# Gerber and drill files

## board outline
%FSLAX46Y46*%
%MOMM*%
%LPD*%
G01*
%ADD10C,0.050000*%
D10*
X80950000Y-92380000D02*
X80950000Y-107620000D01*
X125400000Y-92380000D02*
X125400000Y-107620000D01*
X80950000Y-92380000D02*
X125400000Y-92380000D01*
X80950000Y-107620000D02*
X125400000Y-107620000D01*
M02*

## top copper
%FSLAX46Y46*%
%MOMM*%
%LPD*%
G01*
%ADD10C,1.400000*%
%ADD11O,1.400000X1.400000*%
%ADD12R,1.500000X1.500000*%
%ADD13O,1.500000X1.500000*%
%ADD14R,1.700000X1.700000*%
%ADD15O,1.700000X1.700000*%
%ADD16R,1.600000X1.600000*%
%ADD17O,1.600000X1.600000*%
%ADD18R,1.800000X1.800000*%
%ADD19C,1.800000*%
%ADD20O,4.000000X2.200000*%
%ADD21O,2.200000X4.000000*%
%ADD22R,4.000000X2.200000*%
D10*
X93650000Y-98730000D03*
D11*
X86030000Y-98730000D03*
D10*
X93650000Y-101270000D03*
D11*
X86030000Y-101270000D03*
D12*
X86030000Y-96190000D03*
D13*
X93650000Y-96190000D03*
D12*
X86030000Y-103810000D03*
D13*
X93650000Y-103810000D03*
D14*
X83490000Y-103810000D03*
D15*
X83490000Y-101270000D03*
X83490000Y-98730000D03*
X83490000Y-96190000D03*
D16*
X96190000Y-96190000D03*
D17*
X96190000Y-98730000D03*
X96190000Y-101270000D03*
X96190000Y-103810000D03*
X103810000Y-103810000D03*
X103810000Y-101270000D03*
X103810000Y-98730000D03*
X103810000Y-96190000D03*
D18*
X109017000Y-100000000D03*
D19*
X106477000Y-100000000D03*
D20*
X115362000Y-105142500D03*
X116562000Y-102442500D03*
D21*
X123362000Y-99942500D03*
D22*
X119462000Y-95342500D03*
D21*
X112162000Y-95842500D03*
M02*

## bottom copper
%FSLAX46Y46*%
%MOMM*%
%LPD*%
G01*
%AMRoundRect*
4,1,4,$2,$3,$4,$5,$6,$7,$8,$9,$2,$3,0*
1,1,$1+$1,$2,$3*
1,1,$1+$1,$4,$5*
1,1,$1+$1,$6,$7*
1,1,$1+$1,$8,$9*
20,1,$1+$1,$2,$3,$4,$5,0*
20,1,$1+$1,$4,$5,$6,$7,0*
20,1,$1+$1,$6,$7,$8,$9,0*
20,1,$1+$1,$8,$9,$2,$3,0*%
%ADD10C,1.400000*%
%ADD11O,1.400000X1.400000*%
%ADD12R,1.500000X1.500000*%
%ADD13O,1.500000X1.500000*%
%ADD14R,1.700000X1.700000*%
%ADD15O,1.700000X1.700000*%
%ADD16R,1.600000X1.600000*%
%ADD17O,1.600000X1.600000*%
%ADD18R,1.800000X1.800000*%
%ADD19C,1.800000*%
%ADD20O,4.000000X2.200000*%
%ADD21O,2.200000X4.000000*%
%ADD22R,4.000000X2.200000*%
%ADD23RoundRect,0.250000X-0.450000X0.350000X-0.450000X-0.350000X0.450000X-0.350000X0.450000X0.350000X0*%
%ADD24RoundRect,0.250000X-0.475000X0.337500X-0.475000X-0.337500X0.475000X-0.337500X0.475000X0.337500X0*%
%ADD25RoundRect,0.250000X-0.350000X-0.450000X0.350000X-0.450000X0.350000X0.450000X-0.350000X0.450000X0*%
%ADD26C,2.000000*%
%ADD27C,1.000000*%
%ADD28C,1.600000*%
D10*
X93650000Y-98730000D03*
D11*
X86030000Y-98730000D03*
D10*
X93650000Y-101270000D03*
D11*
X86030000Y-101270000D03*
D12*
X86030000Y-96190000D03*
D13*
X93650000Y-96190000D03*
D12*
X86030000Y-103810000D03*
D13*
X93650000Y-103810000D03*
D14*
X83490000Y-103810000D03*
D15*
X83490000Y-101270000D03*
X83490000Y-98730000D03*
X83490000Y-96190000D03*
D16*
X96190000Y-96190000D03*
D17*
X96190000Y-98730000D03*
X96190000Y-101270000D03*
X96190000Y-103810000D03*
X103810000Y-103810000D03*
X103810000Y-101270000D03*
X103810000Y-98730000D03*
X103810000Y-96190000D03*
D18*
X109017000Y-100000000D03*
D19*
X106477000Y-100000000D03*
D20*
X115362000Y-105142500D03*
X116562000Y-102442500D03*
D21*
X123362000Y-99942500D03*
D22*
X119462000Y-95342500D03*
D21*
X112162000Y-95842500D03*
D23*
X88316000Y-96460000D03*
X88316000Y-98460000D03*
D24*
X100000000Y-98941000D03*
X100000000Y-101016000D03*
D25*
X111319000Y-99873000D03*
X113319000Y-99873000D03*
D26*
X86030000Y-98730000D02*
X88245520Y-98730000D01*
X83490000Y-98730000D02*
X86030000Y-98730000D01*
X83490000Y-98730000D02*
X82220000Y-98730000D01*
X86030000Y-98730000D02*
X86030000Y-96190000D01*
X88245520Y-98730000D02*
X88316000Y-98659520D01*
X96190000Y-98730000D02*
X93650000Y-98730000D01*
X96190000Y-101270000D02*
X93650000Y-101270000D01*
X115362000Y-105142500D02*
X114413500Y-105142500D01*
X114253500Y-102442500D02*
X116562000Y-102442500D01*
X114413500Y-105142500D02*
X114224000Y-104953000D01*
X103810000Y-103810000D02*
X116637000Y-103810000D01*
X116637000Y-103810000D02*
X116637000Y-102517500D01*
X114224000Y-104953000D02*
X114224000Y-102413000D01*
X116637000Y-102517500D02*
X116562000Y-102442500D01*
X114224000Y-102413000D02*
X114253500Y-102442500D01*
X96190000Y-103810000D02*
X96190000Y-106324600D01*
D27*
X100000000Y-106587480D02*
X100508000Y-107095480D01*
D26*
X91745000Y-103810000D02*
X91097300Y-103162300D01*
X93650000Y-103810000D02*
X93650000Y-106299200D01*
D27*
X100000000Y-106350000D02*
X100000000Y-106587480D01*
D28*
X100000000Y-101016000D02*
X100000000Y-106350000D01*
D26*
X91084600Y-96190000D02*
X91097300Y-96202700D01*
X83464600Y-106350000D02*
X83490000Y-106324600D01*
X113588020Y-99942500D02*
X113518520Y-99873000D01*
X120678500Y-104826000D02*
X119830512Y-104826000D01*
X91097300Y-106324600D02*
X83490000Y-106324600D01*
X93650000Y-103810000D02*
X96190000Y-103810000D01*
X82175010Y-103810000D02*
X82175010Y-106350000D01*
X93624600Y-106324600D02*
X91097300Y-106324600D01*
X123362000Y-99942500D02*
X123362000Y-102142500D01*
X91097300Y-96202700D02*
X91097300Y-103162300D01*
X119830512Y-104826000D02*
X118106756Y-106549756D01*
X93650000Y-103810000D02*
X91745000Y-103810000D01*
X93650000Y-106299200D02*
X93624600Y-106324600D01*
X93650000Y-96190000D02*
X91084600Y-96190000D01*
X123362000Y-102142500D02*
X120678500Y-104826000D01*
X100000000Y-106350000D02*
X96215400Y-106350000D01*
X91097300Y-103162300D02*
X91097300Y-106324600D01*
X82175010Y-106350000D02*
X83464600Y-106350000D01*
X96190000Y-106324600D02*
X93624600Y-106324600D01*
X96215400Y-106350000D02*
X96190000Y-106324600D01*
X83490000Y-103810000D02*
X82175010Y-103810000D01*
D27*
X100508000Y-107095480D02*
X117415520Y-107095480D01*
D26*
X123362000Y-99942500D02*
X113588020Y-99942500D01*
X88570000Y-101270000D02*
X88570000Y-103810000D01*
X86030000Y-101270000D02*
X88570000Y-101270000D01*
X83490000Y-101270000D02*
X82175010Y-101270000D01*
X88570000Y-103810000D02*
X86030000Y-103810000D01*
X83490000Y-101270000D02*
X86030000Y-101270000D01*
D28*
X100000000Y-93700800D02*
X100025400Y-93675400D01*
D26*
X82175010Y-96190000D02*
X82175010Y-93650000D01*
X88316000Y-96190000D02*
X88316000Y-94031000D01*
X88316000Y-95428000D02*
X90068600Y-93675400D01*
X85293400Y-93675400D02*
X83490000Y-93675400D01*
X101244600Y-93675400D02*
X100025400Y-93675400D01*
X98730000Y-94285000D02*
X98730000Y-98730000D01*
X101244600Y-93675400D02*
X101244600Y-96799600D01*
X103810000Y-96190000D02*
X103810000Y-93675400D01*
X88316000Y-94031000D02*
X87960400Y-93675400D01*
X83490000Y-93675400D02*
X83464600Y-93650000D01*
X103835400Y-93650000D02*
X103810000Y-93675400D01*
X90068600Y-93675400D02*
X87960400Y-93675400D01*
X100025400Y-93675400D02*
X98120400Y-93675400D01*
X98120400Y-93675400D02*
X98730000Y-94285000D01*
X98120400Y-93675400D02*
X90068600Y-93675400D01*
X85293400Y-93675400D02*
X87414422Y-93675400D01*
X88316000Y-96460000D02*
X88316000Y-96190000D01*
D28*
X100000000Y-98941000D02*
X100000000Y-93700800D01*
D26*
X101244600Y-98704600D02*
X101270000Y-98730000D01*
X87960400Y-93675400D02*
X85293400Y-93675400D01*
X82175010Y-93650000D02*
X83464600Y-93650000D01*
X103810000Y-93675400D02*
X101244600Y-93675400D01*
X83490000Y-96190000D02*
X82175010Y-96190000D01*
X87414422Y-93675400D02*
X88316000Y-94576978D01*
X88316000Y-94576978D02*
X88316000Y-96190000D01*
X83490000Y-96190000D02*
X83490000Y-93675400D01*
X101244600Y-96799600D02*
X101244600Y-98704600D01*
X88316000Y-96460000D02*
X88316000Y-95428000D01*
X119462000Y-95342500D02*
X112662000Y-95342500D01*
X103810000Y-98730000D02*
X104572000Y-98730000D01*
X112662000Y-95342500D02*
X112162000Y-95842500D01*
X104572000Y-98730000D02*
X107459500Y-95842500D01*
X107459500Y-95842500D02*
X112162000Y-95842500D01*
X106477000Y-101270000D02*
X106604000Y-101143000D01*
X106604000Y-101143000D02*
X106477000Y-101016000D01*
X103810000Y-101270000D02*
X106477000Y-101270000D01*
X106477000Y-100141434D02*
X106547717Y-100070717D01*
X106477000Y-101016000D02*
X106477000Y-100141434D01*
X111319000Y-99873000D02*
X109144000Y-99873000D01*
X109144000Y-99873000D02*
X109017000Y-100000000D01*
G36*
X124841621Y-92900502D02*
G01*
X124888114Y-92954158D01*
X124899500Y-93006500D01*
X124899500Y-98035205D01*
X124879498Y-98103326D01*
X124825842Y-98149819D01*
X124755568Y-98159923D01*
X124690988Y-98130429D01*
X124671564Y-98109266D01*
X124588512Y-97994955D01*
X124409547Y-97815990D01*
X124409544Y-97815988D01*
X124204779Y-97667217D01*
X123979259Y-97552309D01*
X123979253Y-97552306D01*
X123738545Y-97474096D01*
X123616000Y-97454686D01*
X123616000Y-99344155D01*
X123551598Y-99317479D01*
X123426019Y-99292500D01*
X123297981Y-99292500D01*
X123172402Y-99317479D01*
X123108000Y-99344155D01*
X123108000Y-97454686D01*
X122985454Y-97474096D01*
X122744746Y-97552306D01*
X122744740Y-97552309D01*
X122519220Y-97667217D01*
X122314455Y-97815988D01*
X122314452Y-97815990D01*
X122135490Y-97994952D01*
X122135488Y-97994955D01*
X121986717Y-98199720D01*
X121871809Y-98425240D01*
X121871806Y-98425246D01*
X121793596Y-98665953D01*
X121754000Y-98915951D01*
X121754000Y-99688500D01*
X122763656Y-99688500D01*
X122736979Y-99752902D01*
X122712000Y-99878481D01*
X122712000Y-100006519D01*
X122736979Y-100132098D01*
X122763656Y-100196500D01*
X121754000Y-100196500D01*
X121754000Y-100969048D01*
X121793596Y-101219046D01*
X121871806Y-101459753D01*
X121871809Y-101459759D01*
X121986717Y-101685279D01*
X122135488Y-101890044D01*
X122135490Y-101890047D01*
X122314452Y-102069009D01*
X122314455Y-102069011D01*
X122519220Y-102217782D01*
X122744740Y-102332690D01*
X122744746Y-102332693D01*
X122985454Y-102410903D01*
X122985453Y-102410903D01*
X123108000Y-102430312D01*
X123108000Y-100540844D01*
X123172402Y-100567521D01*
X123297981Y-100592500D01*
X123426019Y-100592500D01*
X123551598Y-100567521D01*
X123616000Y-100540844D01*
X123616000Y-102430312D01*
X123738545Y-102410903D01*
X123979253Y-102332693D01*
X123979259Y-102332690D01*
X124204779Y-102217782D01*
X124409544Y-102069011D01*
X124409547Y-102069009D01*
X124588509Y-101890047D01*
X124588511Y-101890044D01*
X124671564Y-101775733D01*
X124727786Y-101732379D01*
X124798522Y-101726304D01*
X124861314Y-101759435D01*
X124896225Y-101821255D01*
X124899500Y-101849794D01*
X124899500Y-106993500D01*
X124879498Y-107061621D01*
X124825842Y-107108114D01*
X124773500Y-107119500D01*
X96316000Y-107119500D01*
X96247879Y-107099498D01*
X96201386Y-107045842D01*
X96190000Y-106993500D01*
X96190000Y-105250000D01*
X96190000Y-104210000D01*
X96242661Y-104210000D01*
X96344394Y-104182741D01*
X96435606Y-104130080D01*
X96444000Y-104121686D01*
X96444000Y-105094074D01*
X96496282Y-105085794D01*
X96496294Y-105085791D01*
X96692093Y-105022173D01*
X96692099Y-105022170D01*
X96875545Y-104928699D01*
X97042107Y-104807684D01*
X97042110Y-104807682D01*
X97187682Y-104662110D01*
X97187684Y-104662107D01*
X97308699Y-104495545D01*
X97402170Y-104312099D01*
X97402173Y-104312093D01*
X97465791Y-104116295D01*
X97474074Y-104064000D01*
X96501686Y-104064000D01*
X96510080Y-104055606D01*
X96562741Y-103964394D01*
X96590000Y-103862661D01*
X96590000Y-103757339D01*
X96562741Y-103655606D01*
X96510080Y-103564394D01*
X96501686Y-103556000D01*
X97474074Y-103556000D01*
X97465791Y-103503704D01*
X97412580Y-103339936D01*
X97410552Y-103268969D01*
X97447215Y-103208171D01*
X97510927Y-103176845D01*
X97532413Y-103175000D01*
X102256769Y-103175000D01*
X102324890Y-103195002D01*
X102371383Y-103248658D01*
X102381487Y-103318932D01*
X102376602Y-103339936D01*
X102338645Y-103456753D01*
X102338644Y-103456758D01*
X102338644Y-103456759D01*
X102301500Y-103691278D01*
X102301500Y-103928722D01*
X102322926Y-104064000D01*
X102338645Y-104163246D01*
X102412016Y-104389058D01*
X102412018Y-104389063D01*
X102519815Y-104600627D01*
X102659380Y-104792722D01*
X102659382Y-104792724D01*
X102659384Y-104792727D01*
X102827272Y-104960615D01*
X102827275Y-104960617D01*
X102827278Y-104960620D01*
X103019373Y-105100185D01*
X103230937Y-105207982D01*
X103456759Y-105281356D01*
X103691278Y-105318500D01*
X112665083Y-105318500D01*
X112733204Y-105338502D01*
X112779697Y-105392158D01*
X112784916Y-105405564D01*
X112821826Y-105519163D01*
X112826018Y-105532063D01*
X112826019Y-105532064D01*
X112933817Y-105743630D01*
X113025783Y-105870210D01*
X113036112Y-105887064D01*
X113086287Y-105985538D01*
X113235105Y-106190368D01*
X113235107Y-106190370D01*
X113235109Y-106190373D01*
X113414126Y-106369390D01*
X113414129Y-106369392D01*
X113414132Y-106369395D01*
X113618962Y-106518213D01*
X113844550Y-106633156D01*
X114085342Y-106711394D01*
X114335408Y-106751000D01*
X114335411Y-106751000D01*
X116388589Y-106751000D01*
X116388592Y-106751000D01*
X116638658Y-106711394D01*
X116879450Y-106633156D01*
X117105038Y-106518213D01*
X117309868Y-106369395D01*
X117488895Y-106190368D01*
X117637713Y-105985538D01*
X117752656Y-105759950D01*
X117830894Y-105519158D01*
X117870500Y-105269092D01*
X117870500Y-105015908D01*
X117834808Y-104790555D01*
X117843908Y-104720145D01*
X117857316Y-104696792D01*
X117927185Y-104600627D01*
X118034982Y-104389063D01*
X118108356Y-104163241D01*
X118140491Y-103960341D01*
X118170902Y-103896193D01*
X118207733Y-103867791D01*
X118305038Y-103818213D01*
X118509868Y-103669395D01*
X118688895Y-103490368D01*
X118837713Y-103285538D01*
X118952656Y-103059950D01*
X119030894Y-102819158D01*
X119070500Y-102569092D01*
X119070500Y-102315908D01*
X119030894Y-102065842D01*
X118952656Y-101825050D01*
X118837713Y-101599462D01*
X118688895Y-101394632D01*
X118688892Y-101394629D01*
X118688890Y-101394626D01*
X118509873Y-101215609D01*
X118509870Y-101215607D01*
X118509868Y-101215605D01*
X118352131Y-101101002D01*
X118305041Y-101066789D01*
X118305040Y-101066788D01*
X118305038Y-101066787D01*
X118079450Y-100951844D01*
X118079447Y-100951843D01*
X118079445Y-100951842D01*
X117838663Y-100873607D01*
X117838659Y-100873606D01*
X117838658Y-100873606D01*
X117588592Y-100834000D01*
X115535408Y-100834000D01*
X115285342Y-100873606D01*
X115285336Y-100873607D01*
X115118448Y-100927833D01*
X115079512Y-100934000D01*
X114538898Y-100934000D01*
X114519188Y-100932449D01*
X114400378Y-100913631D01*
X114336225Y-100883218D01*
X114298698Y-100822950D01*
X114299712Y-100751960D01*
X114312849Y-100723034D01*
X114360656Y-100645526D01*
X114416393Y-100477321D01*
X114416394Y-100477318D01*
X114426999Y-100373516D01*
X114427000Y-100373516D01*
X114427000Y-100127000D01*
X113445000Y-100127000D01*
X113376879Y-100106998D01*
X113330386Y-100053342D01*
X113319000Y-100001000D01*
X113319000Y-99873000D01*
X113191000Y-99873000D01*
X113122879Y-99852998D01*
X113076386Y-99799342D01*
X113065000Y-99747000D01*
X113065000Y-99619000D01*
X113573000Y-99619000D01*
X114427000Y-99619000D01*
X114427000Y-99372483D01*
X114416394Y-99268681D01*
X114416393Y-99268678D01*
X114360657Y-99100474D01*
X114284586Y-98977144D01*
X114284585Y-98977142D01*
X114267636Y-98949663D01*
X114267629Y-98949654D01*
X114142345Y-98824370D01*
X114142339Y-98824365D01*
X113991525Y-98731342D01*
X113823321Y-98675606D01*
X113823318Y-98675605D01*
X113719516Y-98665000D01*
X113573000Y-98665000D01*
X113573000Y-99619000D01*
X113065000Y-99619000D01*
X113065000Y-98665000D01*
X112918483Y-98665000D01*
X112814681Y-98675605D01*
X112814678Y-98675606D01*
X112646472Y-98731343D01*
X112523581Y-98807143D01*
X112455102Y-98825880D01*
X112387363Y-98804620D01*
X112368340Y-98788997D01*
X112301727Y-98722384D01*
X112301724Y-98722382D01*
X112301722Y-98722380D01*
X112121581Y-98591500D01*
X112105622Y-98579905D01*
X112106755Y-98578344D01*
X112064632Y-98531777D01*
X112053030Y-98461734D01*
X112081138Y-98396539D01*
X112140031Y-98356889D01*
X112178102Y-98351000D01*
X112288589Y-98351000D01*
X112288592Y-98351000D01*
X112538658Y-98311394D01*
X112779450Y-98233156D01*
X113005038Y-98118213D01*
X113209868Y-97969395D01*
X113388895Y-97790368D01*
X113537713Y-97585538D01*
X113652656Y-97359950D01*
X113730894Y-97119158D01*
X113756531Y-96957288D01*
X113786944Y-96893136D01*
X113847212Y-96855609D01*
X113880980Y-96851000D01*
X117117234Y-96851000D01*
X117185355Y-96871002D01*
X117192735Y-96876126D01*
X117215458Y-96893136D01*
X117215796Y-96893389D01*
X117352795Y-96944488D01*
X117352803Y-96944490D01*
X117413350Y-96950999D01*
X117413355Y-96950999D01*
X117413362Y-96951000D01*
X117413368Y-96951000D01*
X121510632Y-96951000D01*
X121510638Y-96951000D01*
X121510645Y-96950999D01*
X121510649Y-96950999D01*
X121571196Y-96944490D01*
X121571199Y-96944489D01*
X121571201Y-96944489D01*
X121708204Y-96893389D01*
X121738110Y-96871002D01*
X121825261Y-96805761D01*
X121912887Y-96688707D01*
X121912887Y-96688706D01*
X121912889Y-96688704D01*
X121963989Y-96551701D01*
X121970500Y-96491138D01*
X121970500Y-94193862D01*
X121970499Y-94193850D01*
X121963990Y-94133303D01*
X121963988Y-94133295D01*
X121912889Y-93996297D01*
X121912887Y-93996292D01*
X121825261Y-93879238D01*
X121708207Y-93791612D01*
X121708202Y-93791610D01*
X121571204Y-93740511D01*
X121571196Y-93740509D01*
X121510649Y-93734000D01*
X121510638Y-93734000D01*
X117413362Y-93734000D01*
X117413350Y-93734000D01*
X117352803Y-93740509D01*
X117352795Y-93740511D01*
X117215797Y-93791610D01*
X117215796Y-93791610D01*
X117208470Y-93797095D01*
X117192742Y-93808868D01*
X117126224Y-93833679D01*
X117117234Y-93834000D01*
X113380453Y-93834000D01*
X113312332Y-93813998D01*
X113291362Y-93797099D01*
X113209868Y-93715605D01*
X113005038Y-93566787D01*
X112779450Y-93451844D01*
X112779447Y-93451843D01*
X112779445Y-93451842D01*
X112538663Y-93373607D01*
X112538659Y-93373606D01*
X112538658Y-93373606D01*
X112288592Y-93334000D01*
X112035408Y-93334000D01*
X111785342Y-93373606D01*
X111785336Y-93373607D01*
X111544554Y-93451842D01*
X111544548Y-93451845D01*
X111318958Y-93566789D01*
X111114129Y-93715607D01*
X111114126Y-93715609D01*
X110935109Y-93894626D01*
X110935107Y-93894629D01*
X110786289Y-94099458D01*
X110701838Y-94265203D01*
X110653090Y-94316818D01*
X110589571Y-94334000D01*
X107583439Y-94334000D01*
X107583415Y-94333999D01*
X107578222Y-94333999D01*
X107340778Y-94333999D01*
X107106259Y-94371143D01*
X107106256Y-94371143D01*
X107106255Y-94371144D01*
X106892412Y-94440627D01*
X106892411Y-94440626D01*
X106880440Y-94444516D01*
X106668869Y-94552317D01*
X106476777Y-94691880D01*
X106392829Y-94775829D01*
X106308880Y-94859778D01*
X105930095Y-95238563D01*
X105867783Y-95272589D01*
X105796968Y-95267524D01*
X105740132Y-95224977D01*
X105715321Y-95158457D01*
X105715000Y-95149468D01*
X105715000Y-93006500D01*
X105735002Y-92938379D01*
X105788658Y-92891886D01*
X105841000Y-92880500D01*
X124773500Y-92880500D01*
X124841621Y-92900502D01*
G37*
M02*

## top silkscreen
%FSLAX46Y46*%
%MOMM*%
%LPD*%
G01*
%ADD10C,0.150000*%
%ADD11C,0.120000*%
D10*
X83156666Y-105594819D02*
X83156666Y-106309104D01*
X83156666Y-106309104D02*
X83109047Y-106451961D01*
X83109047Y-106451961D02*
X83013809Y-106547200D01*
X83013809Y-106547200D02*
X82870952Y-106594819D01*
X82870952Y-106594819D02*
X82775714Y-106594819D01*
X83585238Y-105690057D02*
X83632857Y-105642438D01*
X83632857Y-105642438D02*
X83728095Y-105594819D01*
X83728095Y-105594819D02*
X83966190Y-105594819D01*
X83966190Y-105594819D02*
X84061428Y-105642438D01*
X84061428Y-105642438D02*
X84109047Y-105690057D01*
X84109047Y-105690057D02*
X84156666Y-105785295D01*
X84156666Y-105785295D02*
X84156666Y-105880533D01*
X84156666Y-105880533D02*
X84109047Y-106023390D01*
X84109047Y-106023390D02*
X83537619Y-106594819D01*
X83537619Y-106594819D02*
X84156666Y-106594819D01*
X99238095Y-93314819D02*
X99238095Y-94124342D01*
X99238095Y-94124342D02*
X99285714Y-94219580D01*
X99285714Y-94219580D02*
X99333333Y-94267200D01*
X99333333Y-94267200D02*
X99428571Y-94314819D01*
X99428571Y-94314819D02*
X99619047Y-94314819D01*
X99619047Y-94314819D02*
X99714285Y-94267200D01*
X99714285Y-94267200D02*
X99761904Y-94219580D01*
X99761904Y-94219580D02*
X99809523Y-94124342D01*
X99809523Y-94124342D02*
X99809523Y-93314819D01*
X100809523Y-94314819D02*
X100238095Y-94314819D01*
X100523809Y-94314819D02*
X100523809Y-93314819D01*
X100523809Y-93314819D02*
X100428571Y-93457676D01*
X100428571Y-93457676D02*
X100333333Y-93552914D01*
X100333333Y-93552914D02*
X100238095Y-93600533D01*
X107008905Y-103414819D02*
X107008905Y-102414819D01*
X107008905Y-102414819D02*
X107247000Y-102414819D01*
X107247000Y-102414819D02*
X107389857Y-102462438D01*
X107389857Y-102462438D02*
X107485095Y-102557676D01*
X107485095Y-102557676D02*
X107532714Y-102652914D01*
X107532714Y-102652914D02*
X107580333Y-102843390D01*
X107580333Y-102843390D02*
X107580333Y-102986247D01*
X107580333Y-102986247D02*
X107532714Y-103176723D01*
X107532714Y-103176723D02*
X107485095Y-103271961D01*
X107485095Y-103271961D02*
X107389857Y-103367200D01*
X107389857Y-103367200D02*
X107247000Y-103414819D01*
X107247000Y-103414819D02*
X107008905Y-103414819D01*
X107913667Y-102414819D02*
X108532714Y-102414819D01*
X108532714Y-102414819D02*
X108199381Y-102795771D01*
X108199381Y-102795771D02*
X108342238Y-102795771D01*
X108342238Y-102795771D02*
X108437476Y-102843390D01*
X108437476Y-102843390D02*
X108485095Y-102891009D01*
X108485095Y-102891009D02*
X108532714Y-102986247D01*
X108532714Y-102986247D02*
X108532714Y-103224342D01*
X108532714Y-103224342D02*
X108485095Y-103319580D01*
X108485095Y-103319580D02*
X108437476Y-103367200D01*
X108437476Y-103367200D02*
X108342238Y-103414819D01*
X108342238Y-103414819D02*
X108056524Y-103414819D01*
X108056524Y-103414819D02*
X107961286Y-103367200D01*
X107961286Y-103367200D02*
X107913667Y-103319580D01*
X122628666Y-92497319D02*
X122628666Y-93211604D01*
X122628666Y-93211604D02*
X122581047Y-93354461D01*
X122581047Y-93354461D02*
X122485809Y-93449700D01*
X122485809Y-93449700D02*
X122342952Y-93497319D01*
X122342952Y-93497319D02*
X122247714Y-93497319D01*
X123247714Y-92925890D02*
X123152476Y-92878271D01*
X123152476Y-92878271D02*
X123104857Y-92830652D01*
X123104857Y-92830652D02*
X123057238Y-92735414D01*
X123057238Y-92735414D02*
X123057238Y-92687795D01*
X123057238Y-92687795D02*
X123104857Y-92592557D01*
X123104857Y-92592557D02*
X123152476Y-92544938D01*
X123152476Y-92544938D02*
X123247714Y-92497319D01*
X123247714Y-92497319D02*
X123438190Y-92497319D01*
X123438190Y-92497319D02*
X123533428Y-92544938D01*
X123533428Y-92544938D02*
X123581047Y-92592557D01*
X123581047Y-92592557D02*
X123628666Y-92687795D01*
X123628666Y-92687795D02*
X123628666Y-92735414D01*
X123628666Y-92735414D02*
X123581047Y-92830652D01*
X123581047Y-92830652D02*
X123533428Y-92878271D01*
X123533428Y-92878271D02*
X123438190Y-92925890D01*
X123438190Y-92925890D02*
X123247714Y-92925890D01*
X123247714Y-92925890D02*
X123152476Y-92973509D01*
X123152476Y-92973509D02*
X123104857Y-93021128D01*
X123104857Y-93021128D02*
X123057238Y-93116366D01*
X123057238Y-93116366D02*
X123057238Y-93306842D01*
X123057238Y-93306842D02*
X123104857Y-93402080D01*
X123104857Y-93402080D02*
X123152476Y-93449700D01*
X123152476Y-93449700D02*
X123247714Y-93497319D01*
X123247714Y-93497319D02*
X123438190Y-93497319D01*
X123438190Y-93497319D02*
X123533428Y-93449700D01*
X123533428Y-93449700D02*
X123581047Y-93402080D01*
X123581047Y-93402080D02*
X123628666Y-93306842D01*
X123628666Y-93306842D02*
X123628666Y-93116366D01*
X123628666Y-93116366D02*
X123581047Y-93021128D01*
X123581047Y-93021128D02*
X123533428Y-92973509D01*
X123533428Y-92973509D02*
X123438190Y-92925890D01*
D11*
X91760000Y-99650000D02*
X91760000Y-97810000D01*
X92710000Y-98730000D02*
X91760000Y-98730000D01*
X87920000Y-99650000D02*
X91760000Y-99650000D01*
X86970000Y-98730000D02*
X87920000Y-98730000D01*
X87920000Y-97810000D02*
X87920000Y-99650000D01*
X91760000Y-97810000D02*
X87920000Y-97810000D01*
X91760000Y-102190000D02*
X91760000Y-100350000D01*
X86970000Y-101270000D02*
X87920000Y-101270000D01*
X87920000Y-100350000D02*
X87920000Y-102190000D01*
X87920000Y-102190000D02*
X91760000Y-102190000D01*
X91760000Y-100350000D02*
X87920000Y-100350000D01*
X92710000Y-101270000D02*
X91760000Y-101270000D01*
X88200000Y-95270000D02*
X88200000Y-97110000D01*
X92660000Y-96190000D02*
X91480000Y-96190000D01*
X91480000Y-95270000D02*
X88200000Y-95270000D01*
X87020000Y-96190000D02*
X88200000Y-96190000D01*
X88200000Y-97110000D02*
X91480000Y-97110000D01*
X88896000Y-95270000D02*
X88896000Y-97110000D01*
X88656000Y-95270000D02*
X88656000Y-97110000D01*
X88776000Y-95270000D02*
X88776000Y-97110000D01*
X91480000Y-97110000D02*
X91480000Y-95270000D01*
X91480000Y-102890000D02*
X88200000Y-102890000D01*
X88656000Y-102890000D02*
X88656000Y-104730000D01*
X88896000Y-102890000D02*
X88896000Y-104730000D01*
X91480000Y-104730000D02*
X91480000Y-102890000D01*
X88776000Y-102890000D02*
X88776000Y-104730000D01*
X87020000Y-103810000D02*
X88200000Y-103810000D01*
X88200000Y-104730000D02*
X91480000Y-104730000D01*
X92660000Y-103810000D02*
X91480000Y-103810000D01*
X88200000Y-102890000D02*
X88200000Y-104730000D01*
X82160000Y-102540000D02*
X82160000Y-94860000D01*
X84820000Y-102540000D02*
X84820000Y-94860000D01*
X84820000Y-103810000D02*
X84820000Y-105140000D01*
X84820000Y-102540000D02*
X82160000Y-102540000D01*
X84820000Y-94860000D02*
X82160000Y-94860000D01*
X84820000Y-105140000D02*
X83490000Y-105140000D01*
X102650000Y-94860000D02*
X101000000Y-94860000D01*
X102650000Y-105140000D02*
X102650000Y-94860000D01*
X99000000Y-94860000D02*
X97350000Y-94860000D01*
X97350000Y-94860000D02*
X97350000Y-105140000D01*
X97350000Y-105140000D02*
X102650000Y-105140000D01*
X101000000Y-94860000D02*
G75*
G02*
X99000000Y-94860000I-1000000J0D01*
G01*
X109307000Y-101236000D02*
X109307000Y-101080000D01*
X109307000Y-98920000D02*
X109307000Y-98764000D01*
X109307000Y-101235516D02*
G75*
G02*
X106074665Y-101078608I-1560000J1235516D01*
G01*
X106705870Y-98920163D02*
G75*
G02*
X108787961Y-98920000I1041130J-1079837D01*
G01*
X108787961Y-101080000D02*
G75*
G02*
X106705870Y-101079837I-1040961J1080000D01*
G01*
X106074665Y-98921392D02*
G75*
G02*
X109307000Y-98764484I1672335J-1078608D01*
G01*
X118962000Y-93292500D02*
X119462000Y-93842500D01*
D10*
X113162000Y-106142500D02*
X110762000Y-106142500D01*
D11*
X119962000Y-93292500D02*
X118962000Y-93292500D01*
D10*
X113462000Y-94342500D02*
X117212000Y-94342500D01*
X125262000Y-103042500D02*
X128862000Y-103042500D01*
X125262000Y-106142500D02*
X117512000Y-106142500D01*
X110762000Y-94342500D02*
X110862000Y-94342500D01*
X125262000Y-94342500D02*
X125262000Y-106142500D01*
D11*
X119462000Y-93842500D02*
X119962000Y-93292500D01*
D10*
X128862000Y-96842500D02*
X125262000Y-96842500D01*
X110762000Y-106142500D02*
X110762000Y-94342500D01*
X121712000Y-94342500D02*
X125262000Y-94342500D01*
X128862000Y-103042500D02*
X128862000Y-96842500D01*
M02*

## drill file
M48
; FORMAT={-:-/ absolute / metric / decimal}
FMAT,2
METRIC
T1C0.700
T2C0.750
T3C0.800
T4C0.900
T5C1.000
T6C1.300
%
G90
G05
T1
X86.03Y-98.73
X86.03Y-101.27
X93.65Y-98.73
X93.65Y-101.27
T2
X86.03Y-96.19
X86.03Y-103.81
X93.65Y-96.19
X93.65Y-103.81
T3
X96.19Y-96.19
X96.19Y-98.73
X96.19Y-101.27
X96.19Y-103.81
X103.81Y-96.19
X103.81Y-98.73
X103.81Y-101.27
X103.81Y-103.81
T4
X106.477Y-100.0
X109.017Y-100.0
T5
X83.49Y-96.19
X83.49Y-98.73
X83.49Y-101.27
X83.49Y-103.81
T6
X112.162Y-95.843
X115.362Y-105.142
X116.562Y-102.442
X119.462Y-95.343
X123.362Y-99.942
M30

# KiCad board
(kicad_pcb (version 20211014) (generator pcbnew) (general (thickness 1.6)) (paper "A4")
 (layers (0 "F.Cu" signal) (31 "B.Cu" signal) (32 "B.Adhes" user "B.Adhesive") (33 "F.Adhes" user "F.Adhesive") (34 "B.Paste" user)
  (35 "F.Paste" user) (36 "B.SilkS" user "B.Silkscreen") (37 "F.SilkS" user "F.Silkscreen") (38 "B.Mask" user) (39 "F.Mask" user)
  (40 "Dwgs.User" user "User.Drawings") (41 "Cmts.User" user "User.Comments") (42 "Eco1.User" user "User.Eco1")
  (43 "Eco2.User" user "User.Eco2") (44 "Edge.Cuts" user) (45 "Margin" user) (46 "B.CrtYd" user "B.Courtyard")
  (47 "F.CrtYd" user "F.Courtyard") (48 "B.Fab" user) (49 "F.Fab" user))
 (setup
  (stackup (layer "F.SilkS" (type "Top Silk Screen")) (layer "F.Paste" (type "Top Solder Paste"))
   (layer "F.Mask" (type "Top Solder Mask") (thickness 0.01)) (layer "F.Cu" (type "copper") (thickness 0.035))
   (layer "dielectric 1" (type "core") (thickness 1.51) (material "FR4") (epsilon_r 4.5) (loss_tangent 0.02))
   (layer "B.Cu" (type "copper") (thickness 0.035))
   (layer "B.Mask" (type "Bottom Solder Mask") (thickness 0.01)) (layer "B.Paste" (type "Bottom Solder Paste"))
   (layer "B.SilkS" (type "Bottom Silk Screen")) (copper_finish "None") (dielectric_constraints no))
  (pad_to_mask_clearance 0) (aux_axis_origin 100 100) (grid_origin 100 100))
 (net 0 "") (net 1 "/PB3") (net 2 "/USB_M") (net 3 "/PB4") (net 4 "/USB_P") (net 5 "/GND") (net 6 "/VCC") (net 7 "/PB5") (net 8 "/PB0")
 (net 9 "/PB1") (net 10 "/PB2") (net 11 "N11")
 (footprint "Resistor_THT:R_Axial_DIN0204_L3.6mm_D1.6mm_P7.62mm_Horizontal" (layer "F.Cu") (at 93.65 98.73 180)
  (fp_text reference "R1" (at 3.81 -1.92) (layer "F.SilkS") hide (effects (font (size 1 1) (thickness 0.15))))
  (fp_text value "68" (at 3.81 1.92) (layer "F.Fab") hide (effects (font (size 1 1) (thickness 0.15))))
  (fp_line (start 1.89 -0.92) (end 1.89 0.92) (layer "F.SilkS") (width 0.12))
  (fp_line (start 0.94 0) (end 1.89 0) (layer "F.SilkS") (width 0.12))
  (fp_line (start 5.73 -0.92) (end 1.89 -0.92) (layer "F.SilkS") (width 0.12))
  (fp_line (start 6.68 0) (end 5.73 0) (layer "F.SilkS") (width 0.12))
  (fp_line (start 5.73 0.92) (end 5.73 -0.92) (layer "F.SilkS") (width 0.12))
  (fp_line (start 1.89 0.92) (end 5.73 0.92) (layer "F.SilkS") (width 0.12))
  (pad "1" thru_hole circle locked (at 0 0 180) (size 1.4 1.4) (drill 0.7) (layers *.Cu *.Mask) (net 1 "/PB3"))
  (pad "2" thru_hole oval locked (at 7.62 0 180) (size 1.4 1.4) (drill 0.7) (layers *.Cu *.Mask) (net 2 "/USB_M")))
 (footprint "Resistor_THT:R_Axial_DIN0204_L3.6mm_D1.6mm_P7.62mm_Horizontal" (layer "F.Cu") (at 93.65 101.27 180)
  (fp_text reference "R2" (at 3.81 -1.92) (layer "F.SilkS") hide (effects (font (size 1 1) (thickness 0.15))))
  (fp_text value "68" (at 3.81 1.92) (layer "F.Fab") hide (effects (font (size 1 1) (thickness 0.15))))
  (fp_line (start 1.89 -0.92) (end 1.89 0.92) (layer "F.SilkS") (width 0.12))
  (fp_line (start 6.68 0) (end 5.73 0) (layer "F.SilkS") (width 0.12))
  (fp_line (start 5.73 0.92) (end 5.73 -0.92) (layer "F.SilkS") (width 0.12))
  (fp_line (start 5.73 -0.92) (end 1.89 -0.92) (layer "F.SilkS") (width 0.12))
  (fp_line (start 1.89 0.92) (end 5.73 0.92) (layer "F.SilkS") (width 0.12))
  (fp_line (start 0.94 0) (end 1.89 0) (layer "F.SilkS") (width 0.12))
  (pad "1" thru_hole circle locked (at 0 0 180) (size 1.4 1.4) (drill 0.7) (layers *.Cu *.Mask) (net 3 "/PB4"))
  (pad "2" thru_hole oval locked (at 7.62 0 180) (size 1.4 1.4) (drill 0.7) (layers *.Cu *.Mask) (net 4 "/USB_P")))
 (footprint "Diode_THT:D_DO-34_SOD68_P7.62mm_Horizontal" (layer "F.Cu") (at 86.03 96.19)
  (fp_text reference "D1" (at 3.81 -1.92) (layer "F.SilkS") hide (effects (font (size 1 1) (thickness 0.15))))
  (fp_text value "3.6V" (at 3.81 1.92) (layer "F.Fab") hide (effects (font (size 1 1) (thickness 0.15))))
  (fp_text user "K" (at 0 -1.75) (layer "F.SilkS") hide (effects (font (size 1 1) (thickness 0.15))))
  (fp_line (start 2.17 -0.92) (end 2.17 0.92) (layer "F.SilkS") (width 0.12))
  (fp_line (start 6.63 0) (end 5.45 0) (layer "F.SilkS") (width 0.12))
  (fp_line (start 5.45 -0.92) (end 2.17 -0.92) (layer "F.SilkS") (width 0.12))
  (fp_line (start 0.99 0) (end 2.17 0) (layer "F.SilkS") (width 0.12))
  (fp_line (start 2.17 0.92) (end 5.45 0.92) (layer "F.SilkS") (width 0.12))
  (fp_line (start 2.866 -0.92) (end 2.866 0.92) (layer "F.SilkS") (width 0.12))
  (fp_line (start 2.626 -0.92) (end 2.626 0.92) (layer "F.SilkS") (width 0.12))
  (fp_line (start 2.746 -0.92) (end 2.746 0.92) (layer "F.SilkS") (width 0.12))
  (fp_line (start 5.45 0.92) (end 5.45 -0.92) (layer "F.SilkS") (width 0.12))
  (pad "1" thru_hole rect locked (at 0 0) (size 1.5 1.5) (drill 0.75) (layers *.Cu *.Mask) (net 2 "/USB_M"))
  (pad "2" thru_hole oval locked (at 7.62 0) (size 1.5 1.5) (drill 0.75) (layers *.Cu *.Mask) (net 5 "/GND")))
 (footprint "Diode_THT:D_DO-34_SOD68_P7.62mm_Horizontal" (layer "F.Cu") (at 86.03 103.81)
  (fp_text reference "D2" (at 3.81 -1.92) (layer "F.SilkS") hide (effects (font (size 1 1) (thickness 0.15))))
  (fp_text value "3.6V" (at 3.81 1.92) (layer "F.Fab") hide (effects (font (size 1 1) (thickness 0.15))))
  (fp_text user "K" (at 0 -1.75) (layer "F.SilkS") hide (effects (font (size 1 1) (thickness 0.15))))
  (fp_line (start 5.45 -0.92) (end 2.17 -0.92) (layer "F.SilkS") (width 0.12))
  (fp_line (start 2.626 -0.92) (end 2.626 0.92) (layer "F.SilkS") (width 0.12))
  (fp_line (start 2.866 -0.92) (end 2.866 0.92) (layer "F.SilkS") (width 0.12))
  (fp_line (start 5.45 0.92) (end 5.45 -0.92) (layer "F.SilkS") (width 0.12))
  (fp_line (start 2.746 -0.92) (end 2.746 0.92) (layer "F.SilkS") (width 0.12))
  (fp_line (start 0.99 0) (end 2.17 0) (layer "F.SilkS") (width 0.12))
  (fp_line (start 2.17 0.92) (end 5.45 0.92) (layer "F.SilkS") (width 0.12))
  (fp_line (start 6.63 0) (end 5.45 0) (layer "F.SilkS") (width 0.12))
  (fp_line (start 2.17 -0.92) (end 2.17 0.92) (layer "F.SilkS") (width 0.12))
  (pad "1" thru_hole rect locked (at 0 0) (size 1.5 1.5) (drill 0.75) (layers *.Cu *.Mask) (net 4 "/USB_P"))
  (pad "2" thru_hole oval locked (at 7.62 0) (size 1.5 1.5) (drill 0.75) (layers *.Cu *.Mask) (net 5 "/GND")))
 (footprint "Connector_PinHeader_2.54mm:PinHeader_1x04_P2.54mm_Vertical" (layer "F.Cu") (at 83.49 103.81 180)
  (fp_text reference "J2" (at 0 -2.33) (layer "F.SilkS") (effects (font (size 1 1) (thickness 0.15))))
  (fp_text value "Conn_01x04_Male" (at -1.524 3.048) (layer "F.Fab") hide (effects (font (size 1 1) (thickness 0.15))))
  (fp_line (start 1.33 1.27) (end 1.33 8.95) (layer "F.SilkS") (width 0.12))
  (fp_line (start -1.33 1.27) (end -1.33 8.95) (layer "F.SilkS") (width 0.12))
  (fp_line (start -1.33 0) (end -1.33 -1.33) (layer "F.SilkS") (width 0.12))
  (fp_line (start -1.33 1.27) (end 1.33 1.27) (layer "F.SilkS") (width 0.12))
  (fp_line (start -1.33 8.95) (end 1.33 8.95) (layer "F.SilkS") (width 0.12))
  (fp_line (start -1.33 -1.33) (end 0 -1.33) (layer "F.SilkS") (width 0.12))
  (pad "1" thru_hole rect locked (at 0 0 180) (size 1.7 1.7) (drill 1) (layers *.Cu *.Mask) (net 5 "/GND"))
  (pad "2" thru_hole oval locked (at 0 2.54 180) (size 1.7 1.7) (drill 1) (layers *.Cu *.Mask) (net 4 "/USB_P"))
  (pad "3" thru_hole oval locked (at 0 5.08 180) (size 1.7 1.7) (drill 1) (layers *.Cu *.Mask) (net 2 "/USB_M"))
  (pad "4" thru_hole oval locked (at 0 7.62 180) (size 1.7 1.7) (drill 1) (layers *.Cu *.Mask) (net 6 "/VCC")))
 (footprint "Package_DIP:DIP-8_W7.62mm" (layer "F.Cu") (at 96.19 96.19)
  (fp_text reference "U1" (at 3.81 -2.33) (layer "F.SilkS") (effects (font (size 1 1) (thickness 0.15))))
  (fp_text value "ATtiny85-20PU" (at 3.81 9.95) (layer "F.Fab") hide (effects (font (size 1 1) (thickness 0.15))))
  (fp_line (start 6.46 -1.33) (end 4.81 -1.33) (layer "F.SilkS") (width 0.12))
  (fp_line (start 6.46 8.95) (end 6.46 -1.33) (layer "F.SilkS") (width 0.12))
  (fp_line (start 2.81 -1.33) (end 1.16 -1.33) (layer "F.SilkS") (width 0.12))
  (fp_line (start 1.16 -1.33) (end 1.16 8.95) (layer "F.SilkS") (width 0.12))
  (fp_line (start 1.16 8.95) (end 6.46 8.95) (layer "F.SilkS") (width 0.12))
  (fp_arc (start 4.81 -1.33) (mid 3.81 -0.33) (end 2.81 -1.33) (layer "F.SilkS") (width 0.12))
  (pad "1" thru_hole rect locked (at 0 0) (size 1.6 1.6) (drill 0.8) (layers *.Cu *.Mask) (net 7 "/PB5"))
  (pad "2" thru_hole oval locked (at 0 2.54) (size 1.6 1.6) (drill 0.8) (layers *.Cu *.Mask) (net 1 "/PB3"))
  (pad "3" thru_hole oval locked (at 0 5.08) (size 1.6 1.6) (drill 0.8) (layers *.Cu *.Mask) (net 3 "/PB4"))
  (pad "4" thru_hole oval locked (at 0 7.62) (size 1.6 1.6) (drill 0.8) (layers *.Cu *.Mask) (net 5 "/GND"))
  (pad "5" thru_hole oval locked (at 7.62 7.62) (size 1.6 1.6) (drill 0.8) (layers *.Cu *.Mask) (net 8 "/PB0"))
  (pad "6" thru_hole oval locked (at 7.62 5.08) (size 1.6 1.6) (drill 0.8) (layers *.Cu *.Mask) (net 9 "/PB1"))
  (pad "7" thru_hole oval locked (at 7.62 2.54) (size 1.6 1.6) (drill 0.8) (layers *.Cu *.Mask) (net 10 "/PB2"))
  (pad "8" thru_hole oval locked (at 7.62 0) (size 1.6 1.6) (drill 0.8) (layers *.Cu *.Mask) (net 6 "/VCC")))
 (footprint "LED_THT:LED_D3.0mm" (layer "F.Cu") (at 109.017 100 180)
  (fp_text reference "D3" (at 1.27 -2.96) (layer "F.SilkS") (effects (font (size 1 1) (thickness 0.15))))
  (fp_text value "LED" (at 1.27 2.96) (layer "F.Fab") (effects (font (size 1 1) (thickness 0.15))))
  (fp_line (start -0.29 -1.236) (end -0.29 -1.08) (layer "F.SilkS") (width 0.12))
  (fp_line (start -0.29 1.08) (end -0.29 1.236) (layer "F.SilkS") (width 0.12))
  (fp_arc (start -0.29 -1.235516) (mid 1.366487 -1.987659) (end 2.942335 -1.078608) (layer "F.SilkS") (width 0.12))
  (fp_arc (start 2.31113 1.079837) (mid 1.270117 1.5) (end 0.229039 1.08) (layer "F.SilkS") (width 0.12))
  (fp_arc (start 0.229039 -1.08) (mid 1.270117 -1.5) (end 2.31113 -1.079837) (layer "F.SilkS") (width 0.12))
  (fp_arc (start 2.942335 1.078608) (mid 1.366487 1.987659) (end -0.29 1.235516) (layer "F.SilkS") (width 0.12))
  (pad "1" thru_hole rect (at 0 0 180) (size 1.8 1.8) (drill 0.9) (layers *.Cu *.Mask) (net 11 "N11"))
  (pad "2" thru_hole circle (at 2.54 0 180) (size 1.8 1.8) (drill 0.9) (layers *.Cu *.Mask) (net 9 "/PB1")))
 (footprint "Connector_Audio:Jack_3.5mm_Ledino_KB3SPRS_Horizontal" (layer "F.Cu") (at 119.462 95.3425 180)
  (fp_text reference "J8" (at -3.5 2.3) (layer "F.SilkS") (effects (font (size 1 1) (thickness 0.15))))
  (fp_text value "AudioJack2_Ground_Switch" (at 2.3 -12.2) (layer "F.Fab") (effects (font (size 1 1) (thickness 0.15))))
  (fp_line (start 0.5 2.05) (end 0 1.5) (layer "F.SilkS") (width 0.12))
  (fp_line (start 6.3 -10.8) (end 8.7 -10.8) (layer "F.SilkS") (width 0.15))
  (fp_line (start -0.5 2.05) (end 0.5 2.05) (layer "F.SilkS") (width 0.12))
  (fp_line (start 6 1) (end 2.25 1) (layer "F.SilkS") (width 0.15))
  (fp_line (start -5.8 -7.7) (end -9.4 -7.7) (layer "F.SilkS") (width 0.15))
  (fp_line (start -5.8 -10.8) (end 1.95 -10.8) (layer "F.SilkS") (width 0.15))
  (fp_line (start 8.7 1) (end 8.6 1) (layer "F.SilkS") (width 0.15))
  (fp_line (start -5.8 1) (end -5.8 -10.8) (layer "F.SilkS") (width 0.15))
  (fp_line (start 0 1.5) (end -0.5 2.05) (layer "F.SilkS") (width 0.12))
  (fp_line (start -9.4 -1.5) (end -5.8 -1.5) (layer "F.SilkS") (width 0.15))
  (fp_line (start 8.7 -10.8) (end 8.7 1) (layer "F.SilkS") (width 0.15))
  (fp_line (start -2.25 1) (end -5.8 1) (layer "F.SilkS") (width 0.15))
  (fp_line (start -9.4 -7.7) (end -9.4 -1.5) (layer "F.SilkS") (width 0.15))
  (pad "R" thru_hole oval (at 4.1 -9.8 180) (size 4 2.2) (drill 1.3) (layers *.Cu *.Mask) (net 8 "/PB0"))
  (pad "RN" thru_hole oval (at 2.9 -7.1 180) (size 4 2.2) (drill 1.3) (layers *.Cu *.Mask) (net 8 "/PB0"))
  (pad "S" thru_hole oval (at -3.9 -4.6 180) (size 2.2 4) (drill 1.3) (layers *.Cu *.Mask) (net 5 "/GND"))
  (pad "T" thru_hole rect (at 0 0 180) (size 4 2.2) (drill 1.3) (layers *.Cu *.Mask) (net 10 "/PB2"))
  (pad "TN" thru_hole oval (at 7.3 -0.5 270) (size 4 2.2) (drill 1.3) (layers *.Cu *.Mask) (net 10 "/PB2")))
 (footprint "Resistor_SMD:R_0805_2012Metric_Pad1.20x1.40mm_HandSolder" (layer "B.Cu") (at 88.316 97.46 -90)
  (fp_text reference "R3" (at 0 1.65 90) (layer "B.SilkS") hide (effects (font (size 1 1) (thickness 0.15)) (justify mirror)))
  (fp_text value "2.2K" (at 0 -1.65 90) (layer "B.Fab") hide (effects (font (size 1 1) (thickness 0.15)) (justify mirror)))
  (pad "1" smd roundrect locked (at -1 0 270) (size 1.2 1.4) (layers "B.Cu" "B.Paste" "B.Mask") (roundrect_rratio 0.2083333333)
   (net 6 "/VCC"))
  (pad "2" smd roundrect locked (at 1 0 270) (size 1.2 1.4) (layers "B.Cu" "B.Paste" "B.Mask") (roundrect_rratio 0.2083333333)
   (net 2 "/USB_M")))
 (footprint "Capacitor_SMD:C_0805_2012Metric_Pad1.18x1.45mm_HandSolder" (layer "B.Cu") (at 100 99.9785 -90)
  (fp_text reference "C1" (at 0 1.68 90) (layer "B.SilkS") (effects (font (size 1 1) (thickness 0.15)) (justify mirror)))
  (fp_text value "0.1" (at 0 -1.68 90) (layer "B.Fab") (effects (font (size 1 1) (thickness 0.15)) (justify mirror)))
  (pad "1" smd roundrect locked (at -1.0375 0 270) (size 1.175 1.45) (layers "B.Cu" "B.Paste" "B.Mask") (roundrect_rratio 0.2127659574)
   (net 6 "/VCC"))
  (pad "2" smd roundrect locked (at 1.0375 0 270) (size 1.175 1.45) (layers "B.Cu" "B.Paste" "B.Mask") (roundrect_rratio 0.2127659574)
   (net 5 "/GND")))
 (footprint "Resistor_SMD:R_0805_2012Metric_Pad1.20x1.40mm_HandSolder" (layer "B.Cu") (at 112.319 99.873)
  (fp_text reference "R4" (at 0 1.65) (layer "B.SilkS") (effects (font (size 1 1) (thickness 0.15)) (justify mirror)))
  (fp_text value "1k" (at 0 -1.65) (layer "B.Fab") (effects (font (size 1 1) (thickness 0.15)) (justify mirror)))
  (pad "1" smd roundrect (at -1 0) (size 1.2 1.4) (layers "B.Cu" "B.Paste" "B.Mask") (roundrect_rratio 0.208333) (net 11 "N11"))
  (pad "2" smd roundrect (at 1 0) (size 1.2 1.4) (layers "B.Cu" "B.Paste" "B.Mask") (roundrect_rratio 0.208333) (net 5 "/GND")))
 (gr_line (start 80.95 92.38) (end 80.95 107.62) (layer "Edge.Cuts") (width 0.05))
 (gr_line (start 125.4 92.38) (end 125.4 107.62) (layer "Edge.Cuts") (width 0.05))
 (gr_line (start 80.95 92.38) (end 125.4 92.38) (layer "Edge.Cuts") (width 0.05))
 (gr_line (start 80.95 107.62) (end 125.4 107.62) (layer "Edge.Cuts") (width 0.05))
 (segment (start 86.03 98.73) (end 88.24552 98.73) (width 2) (layer "B.Cu") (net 2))
 (segment (start 83.49 98.73) (end 86.03 98.73) (width 2) (layer "B.Cu") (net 2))
 (segment (start 83.49 98.73) (end 82.22 98.73) (width 2) (layer "B.Cu") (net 2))
 (segment (start 86.03 98.73) (end 86.03 96.19) (width 2) (layer "B.Cu") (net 2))
 (segment (start 88.24552 98.73) (end 88.316 98.65952) (width 2) (layer "B.Cu") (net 2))
 (segment (start 96.19 98.73) (end 93.65 98.73) (width 2) (layer "B.Cu") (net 1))
 (segment (start 96.19 101.27) (end 93.65 101.27) (width 2) (layer "B.Cu") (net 3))
 (segment (start 115.362 105.1425) (end 114.4135 105.1425) (width 2) (layer "B.Cu") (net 8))
 (segment (start 114.2535 102.4425) (end 116.562 102.4425) (width 2) (layer "B.Cu") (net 8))
 (segment (start 114.4135 105.1425) (end 114.224 104.953) (width 2) (layer "B.Cu") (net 8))
 (segment (start 103.81 103.81) (end 116.637 103.81) (width 2) (layer "B.Cu") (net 8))
 (segment (start 116.637 103.81) (end 116.637 102.5175) (width 2) (layer "B.Cu") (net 8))
 (segment (start 114.224 104.953) (end 114.224 102.413) (width 2) (layer "B.Cu") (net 8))
 (segment (start 116.637 102.5175) (end 116.562 102.4425) (width 2) (layer "B.Cu") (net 8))
 (segment (start 114.224 102.413) (end 114.2535 102.4425) (width 2) (layer "B.Cu") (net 8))
 (segment (start 96.19 103.81) (end 96.19 106.3246) (width 2) (layer "B.Cu") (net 5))
 (segment (start 100 106.58748) (end 100.508 107.09548) (width 1) (layer "B.Cu") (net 5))
 (segment (start 91.745 103.81) (end 91.0973 103.1623) (width 2) (layer "B.Cu") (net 5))
 (segment (start 93.65 103.81) (end 93.65 106.2992) (width 2) (layer "B.Cu") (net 5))
 (segment (start 100 106.35) (end 100 106.58748) (width 1) (layer "B.Cu") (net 5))
 (segment (start 100 101.016) (end 100 106.35) (width 1.6) (layer "B.Cu") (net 5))
 (segment (start 91.0846 96.19) (end 91.0973 96.2027) (width 2) (layer "B.Cu") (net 5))
 (segment (start 83.4646 106.35) (end 83.49 106.3246) (width 2) (layer "B.Cu") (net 5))
 (segment (start 113.58802 99.9425) (end 113.51852 99.873) (width 2) (layer "B.Cu") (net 5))
 (segment (start 120.6785 104.826) (end 119.830512 104.826) (width 2) (layer "B.Cu") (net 5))
 (segment (start 91.0973 106.3246) (end 83.49 106.3246) (width 2) (layer "B.Cu") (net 5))
 (segment (start 93.65 103.81) (end 96.19 103.81) (width 2) (layer "B.Cu") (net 5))
 (segment (start 82.17501 103.81) (end 82.17501 106.35) (width 2) (layer "B.Cu") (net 5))
 (segment (start 93.6246 106.3246) (end 91.0973 106.3246) (width 2) (layer "B.Cu") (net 5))
 (segment (start 123.362 99.9425) (end 123.362 102.1425) (width 2) (layer "B.Cu") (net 5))
 (segment (start 91.0973 96.2027) (end 91.0973 103.1623) (width 2) (layer "B.Cu") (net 5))
 (segment (start 119.830512 104.826) (end 118.106756 106.549756) (width 2) (layer "B.Cu") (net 5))
 (segment (start 93.65 103.81) (end 91.745 103.81) (width 2) (layer "B.Cu") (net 5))
 (segment (start 93.65 106.2992) (end 93.6246 106.3246) (width 2) (layer "B.Cu") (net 5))
 (segment (start 93.65 96.19) (end 91.0846 96.19) (width 2) (layer "B.Cu") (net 5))
 (segment (start 123.362 102.1425) (end 120.6785 104.826) (width 2) (layer "B.Cu") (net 5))
 (segment (start 100 106.35) (end 96.2154 106.35) (width 2) (layer "B.Cu") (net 5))
 (segment (start 91.0973 103.1623) (end 91.0973 106.3246) (width 2) (layer "B.Cu") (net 5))
 (segment (start 82.17501 106.35) (end 83.4646 106.35) (width 2) (layer "B.Cu") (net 5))
 (segment (start 96.19 106.3246) (end 93.6246 106.3246) (width 2) (layer "B.Cu") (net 5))
 (segment (start 96.2154 106.35) (end 96.19 106.3246) (width 2) (layer "B.Cu") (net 5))
 (segment (start 83.49 103.81) (end 82.17501 103.81) (width 2) (layer "B.Cu") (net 5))
 (segment (start 100.508 107.09548) (end 117.41552 107.09548) (width 1) (layer "B.Cu") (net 5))
 (segment (start 123.362 99.9425) (end 113.58802 99.9425) (width 2) (layer "B.Cu") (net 5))
 (segment (start 88.57 101.27) (end 88.57 103.81) (width 2) (layer "B.Cu") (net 4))
 (segment (start 86.03 101.27) (end 88.57 101.27) (width 2) (layer "B.Cu") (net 4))
 (segment (start 83.49 101.27) (end 82.17501 101.27) (width 2) (layer "B.Cu") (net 4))
 (segment (start 88.57 103.81) (end 86.03 103.81) (width 2) (layer "B.Cu") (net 4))
 (segment (start 83.49 101.27) (end 86.03 101.27) (width 2) (layer "B.Cu") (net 4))
 (segment (start 100 93.7008) (end 100.0254 93.6754) (width 1.6) (layer "B.Cu") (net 6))
 (segment (start 82.17501 96.19) (end 82.17501 93.65) (width 2) (layer "B.Cu") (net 6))
 (segment (start 88.316 96.19) (end 88.316 94.031) (width 2) (layer "B.Cu") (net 6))
 (segment (start 88.316 95.428) (end 90.0686 93.6754) (width 2) (layer "B.Cu") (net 6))
 (segment (start 85.2934 93.6754) (end 83.49 93.6754) (width 2) (layer "B.Cu") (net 6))
 (segment (start 101.2446 93.6754) (end 100.0254 93.6754) (width 2) (layer "B.Cu") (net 6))
 (segment (start 98.73 94.285) (end 98.73 98.73) (width 2) (layer "B.Cu") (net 6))
 (segment (start 101.2446 93.6754) (end 101.2446 96.7996) (width 2) (layer "B.Cu") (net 6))
 (segment (start 103.81 96.19) (end 103.81 93.6754) (width 2) (layer "B.Cu") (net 6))
 (segment (start 88.316 94.031) (end 87.9604 93.6754) (width 2) (layer "B.Cu") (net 6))
 (segment (start 83.49 93.6754) (end 83.4646 93.65) (width 2) (layer "B.Cu") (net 6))
 (segment (start 103.8354 93.65) (end 103.81 93.6754) (width 2) (layer "B.Cu") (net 6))
 (segment (start 90.0686 93.6754) (end 87.9604 93.6754) (width 2) (layer "B.Cu") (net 6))
 (segment (start 100.0254 93.6754) (end 98.1204 93.6754) (width 2) (layer "B.Cu") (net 6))
 (segment (start 98.1204 93.6754) (end 98.73 94.285) (width 2) (layer "B.Cu") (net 6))
 (segment (start 98.1204 93.6754) (end 90.0686 93.6754) (width 2) (layer "B.Cu") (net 6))
 (segment (start 85.2934 93.6754) (end 87.414422 93.6754) (width 2) (layer "B.Cu") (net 6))
 (segment (start 88.316 96.46) (end 88.316 96.19) (width 2) (layer "B.Cu") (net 6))
 (segment (start 100 98.941) (end 100 93.7008) (width 1.6) (layer "B.Cu") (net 6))
 (segment (start 101.2446 98.7046) (end 101.27 98.73) (width 2) (layer "B.Cu") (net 6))
 (segment (start 87.9604 93.6754) (end 85.2934 93.6754) (width 2) (layer "B.Cu") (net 6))
 (segment (start 82.17501 93.65) (end 83.4646 93.65) (width 2) (layer "B.Cu") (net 6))
 (segment (start 103.81 93.6754) (end 101.2446 93.6754) (width 2) (layer "B.Cu") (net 6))
 (segment (start 83.49 96.19) (end 82.17501 96.19) (width 2) (layer "B.Cu") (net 6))
 (segment (start 87.414422 93.6754) (end 88.316 94.576978) (width 2) (layer "B.Cu") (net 6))
 (segment (start 88.316 94.576978) (end 88.316 96.19) (width 2) (layer "B.Cu") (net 6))
 (segment (start 83.49 96.19) (end 83.49 93.6754) (width 2) (layer "B.Cu") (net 6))
 (segment (start 101.2446 96.7996) (end 101.2446 98.7046) (width 2) (layer "B.Cu") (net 6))
 (segment (start 88.316 96.46) (end 88.316 95.428) (width 2) (layer "B.Cu") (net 6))
 (segment (start 119.462 95.3425) (end 112.662 95.3425) (width 2) (layer "B.Cu") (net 10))
 (segment (start 103.81 98.73) (end 104.572 98.73) (width 2) (layer "B.Cu") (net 10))
 (segment (start 112.662 95.3425) (end 112.162 95.8425) (width 2) (layer "B.Cu") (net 10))
 (segment (start 104.572 98.73) (end 107.4595 95.8425) (width 2) (layer "B.Cu") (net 10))
 (segment (start 107.4595 95.8425) (end 112.162 95.8425) (width 2) (layer "B.Cu") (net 10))
 (segment (start 106.477 101.27) (end 106.604 101.143) (width 2) (layer "B.Cu") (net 9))
 (segment (start 106.604 101.143) (end 106.477 101.016) (width 2) (layer "B.Cu") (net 9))
 (segment (start 103.81 101.27) (end 106.477 101.27) (width 2) (layer "B.Cu") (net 9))
 (segment (start 106.477 100.141434) (end 106.547717 100.070717) (width 2) (layer "B.Cu") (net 9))
 (segment (start 106.477 101.016) (end 106.477 100.141434) (width 2) (layer "B.Cu") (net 9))
 (segment (start 111.319 99.873) (end 109.144 99.873) (width 2) (layer "B.Cu") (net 11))
 (segment (start 109.144 99.873) (end 109.017 100) (width 2) (layer "B.Cu") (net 11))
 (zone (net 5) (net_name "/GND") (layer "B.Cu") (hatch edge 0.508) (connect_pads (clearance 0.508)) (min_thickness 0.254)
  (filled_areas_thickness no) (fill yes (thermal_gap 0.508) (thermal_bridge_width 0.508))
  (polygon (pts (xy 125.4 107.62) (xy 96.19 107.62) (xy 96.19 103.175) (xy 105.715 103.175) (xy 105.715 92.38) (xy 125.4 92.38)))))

